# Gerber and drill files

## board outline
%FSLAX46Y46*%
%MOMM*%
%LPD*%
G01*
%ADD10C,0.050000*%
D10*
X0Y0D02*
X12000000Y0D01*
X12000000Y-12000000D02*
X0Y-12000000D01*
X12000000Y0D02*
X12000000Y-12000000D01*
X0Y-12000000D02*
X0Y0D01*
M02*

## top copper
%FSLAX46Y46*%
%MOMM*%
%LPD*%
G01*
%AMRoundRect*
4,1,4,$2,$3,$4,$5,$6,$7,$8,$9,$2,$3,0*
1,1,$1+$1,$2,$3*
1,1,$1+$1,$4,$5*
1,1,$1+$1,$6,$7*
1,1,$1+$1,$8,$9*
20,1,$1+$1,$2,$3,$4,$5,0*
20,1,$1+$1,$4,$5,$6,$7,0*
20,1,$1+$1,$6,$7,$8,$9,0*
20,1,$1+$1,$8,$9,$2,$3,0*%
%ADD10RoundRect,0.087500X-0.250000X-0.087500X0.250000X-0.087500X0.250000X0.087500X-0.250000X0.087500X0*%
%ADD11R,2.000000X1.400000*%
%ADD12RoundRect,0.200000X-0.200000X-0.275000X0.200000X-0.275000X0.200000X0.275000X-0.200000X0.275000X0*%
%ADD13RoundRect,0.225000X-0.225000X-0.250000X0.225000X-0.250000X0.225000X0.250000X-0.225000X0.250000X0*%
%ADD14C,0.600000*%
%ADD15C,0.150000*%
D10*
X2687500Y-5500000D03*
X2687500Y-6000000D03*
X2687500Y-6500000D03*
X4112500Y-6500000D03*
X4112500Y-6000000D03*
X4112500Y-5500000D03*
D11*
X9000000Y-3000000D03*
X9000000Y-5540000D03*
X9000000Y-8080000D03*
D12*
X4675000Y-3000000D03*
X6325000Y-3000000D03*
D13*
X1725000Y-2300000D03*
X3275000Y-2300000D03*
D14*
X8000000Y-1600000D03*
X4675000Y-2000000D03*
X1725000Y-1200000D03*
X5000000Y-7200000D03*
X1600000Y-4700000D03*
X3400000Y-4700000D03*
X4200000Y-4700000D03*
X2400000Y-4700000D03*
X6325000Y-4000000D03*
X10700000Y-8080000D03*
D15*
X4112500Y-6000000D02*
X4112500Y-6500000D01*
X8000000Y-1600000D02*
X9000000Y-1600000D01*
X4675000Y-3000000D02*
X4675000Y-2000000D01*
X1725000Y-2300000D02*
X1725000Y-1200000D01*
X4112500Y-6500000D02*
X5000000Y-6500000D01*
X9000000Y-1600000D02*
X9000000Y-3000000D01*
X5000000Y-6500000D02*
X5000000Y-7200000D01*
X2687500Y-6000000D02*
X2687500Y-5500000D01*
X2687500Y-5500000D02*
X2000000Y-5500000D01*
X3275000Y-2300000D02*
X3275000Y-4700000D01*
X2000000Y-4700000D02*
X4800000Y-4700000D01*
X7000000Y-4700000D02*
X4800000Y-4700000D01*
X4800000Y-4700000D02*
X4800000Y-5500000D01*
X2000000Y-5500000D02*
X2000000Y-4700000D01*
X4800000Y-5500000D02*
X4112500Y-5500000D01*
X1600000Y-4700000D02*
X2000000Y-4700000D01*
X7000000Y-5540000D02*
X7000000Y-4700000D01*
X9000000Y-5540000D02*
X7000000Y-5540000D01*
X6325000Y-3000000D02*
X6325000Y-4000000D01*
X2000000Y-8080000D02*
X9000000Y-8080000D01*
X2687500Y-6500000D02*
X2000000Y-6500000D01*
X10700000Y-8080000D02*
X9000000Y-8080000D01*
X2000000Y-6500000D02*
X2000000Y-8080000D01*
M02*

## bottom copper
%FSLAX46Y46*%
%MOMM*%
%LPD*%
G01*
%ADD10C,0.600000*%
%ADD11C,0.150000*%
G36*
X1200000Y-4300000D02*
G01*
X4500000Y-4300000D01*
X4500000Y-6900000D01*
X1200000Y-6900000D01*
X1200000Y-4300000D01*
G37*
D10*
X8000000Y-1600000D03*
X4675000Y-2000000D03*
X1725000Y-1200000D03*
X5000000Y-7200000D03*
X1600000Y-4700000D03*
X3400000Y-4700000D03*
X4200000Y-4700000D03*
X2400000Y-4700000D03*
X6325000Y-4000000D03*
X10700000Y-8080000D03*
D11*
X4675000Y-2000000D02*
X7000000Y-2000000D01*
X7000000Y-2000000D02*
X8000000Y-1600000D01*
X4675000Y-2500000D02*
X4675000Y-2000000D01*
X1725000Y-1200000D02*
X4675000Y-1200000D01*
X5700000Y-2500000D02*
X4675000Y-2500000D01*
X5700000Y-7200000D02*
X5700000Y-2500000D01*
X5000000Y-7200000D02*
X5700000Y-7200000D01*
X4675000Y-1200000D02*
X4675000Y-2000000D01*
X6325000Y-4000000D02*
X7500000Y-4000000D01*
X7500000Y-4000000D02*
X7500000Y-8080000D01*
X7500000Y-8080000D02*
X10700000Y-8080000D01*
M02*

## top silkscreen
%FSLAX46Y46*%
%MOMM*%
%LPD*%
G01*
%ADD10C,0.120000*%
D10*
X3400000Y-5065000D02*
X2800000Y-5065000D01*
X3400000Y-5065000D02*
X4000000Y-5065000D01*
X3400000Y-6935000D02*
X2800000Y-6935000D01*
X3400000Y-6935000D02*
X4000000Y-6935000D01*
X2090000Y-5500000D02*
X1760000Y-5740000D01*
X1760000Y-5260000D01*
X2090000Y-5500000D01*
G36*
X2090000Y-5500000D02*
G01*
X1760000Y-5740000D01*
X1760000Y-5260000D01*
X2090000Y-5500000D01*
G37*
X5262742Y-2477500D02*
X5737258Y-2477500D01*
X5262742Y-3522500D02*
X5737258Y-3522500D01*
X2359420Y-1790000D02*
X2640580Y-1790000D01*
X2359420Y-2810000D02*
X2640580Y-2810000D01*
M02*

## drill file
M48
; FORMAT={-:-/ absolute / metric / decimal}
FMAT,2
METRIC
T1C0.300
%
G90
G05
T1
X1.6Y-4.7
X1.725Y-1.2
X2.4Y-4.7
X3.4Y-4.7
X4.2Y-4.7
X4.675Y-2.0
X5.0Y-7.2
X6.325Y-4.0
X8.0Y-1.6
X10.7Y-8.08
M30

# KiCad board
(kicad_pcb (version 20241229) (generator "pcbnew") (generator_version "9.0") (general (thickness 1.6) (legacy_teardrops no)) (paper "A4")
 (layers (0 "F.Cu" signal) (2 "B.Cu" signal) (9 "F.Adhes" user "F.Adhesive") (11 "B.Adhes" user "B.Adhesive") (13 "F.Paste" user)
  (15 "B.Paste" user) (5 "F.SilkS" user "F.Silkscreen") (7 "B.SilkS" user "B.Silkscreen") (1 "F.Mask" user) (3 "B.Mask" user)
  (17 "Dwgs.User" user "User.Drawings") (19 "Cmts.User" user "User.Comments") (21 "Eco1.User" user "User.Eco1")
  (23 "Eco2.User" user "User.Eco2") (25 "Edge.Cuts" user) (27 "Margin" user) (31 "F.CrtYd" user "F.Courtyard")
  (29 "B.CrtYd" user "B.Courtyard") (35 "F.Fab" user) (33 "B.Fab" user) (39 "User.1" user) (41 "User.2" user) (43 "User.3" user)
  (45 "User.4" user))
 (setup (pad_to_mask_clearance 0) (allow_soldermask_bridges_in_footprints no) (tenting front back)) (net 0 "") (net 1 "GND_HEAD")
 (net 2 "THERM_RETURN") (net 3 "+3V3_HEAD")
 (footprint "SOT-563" (layer "F.Cu") (at 3.4 6)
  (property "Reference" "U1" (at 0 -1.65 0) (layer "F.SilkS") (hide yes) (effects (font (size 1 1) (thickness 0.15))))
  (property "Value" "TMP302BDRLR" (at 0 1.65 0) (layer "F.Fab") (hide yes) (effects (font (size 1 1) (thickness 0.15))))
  (fp_line (start 0 -0.935) (end -0.6 -0.935) (stroke (width 0.12) (type solid)) (layer "F.SilkS"))
  (fp_line (start 0 -0.935) (end 0.6 -0.935) (stroke (width 0.12) (type solid)) (layer "F.SilkS"))
  (fp_line (start 0 0.935) (end -0.6 0.935) (stroke (width 0.12) (type solid)) (layer "F.SilkS"))
  (fp_line (start 0 0.935) (end 0.6 0.935) (stroke (width 0.12) (type solid)) (layer "F.SilkS"))
  (fp_poly (pts (xy -1.31 -0.5) (xy -1.64 -0.26) (xy -1.64 -0.74)) (stroke (width 0.12) (type solid)) (fill yes) (layer "F.SilkS"))
  (pad "1" smd roundrect (at -0.7125 -0.5) (size 0.675 0.35) (layers "F.Cu" "F.Mask" "F.Paste") (roundrect_rratio 0.25) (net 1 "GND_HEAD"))
  (pad "2" smd roundrect (at -0.7125 0) (size 0.675 0.35) (layers "F.Cu" "F.Mask" "F.Paste") (roundrect_rratio 0.25) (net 1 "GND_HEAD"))
  (pad "3" smd roundrect (at -0.7125 0.5) (size 0.675 0.35) (layers "F.Cu" "F.Mask" "F.Paste") (roundrect_rratio 0.25)
   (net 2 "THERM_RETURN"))
  (pad "4" smd roundrect (at 0.7125 0.5) (size 0.675 0.35) (layers "F.Cu" "F.Mask" "F.Paste") (roundrect_rratio 0.25) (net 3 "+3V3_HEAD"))
  (pad "5" smd roundrect (at 0.7125 0) (size 0.675 0.35) (layers "F.Cu" "F.Mask" "F.Paste") (roundrect_rratio 0.25) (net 3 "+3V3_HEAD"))
  (pad "6" smd roundrect (at 0.7125 -0.5) (size 0.675 0.35) (layers "F.Cu" "F.Mask" "F.Paste") (roundrect_rratio 0.25) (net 1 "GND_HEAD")))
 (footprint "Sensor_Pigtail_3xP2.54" (layer "F.Cu") (at 9 3)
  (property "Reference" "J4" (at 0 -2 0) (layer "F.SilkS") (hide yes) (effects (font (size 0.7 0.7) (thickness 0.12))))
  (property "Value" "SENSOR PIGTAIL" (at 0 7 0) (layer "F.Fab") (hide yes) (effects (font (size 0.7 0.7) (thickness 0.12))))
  (pad "1" smd rect (at 0 0) (size 2 1.4) (layers "F.Cu" "F.Mask" "F.Paste") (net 3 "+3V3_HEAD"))
  (pad "2" smd rect (at 0 2.54) (size 2 1.4) (layers "F.Cu" "F.Mask" "F.Paste") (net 1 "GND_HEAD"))
  (pad "3" smd rect (at 0 5.08) (size 2 1.4) (layers "F.Cu" "F.Mask" "F.Paste") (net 2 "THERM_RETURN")))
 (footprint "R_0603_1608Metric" (layer "F.Cu") (at 5.5 3)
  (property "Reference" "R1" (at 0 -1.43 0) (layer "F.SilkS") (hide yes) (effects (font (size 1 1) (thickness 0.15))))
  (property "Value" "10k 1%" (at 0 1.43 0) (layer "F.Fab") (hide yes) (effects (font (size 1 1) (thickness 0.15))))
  (fp_line (start -0.237258 -0.5225) (end 0.237258 -0.5225) (stroke (width 0.12) (type solid)) (layer "F.SilkS"))
  (fp_line (start -0.237258 0.5225) (end 0.237258 0.5225) (stroke (width 0.12) (type solid)) (layer "F.SilkS"))
  (pad "1" smd roundrect (at -0.825 0) (size 0.8 0.95) (layers "F.Cu" "F.Mask" "F.Paste") (roundrect_rratio 0.25) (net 3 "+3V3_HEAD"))
  (pad "2" smd roundrect (at 0.825 0) (size 0.8 0.95) (layers "F.Cu" "F.Mask" "F.Paste") (roundrect_rratio 0.25) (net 2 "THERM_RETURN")))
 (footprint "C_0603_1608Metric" (layer "F.Cu") (at 2.5 2.3)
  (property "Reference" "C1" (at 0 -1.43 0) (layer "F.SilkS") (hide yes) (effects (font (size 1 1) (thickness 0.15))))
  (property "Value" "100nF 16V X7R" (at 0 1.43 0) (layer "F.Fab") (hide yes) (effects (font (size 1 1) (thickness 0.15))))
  (fp_line (start -0.14058 -0.51) (end 0.14058 -0.51) (stroke (width 0.12) (type solid)) (layer "F.SilkS"))
  (fp_line (start -0.14058 0.51) (end 0.14058 0.51) (stroke (width 0.12) (type solid)) (layer "F.SilkS"))
  (pad "1" smd roundrect (at -0.775 0) (size 0.9 0.95) (layers "F.Cu" "F.Mask" "F.Paste") (roundrect_rratio 0.25) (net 3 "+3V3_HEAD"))
  (pad "2" smd roundrect (at 0.775 0) (size 0.9 0.95) (layers "F.Cu" "F.Mask" "F.Paste") (roundrect_rratio 0.25) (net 1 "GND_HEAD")))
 (gr_rect (start 1.2 4.3) (end 4.5 6.9) (stroke (width 0) (type default)) (fill yes) (layer "B.Cu") (net 1))
 (gr_line (start 0 0) (end 12 0) (stroke (width 0.05) (type default)) (layer "Edge.Cuts"))
 (gr_line (start 12 12) (end 0 12) (stroke (width 0.05) (type default)) (layer "Edge.Cuts"))
 (gr_line (start 12 0) (end 12 12) (stroke (width 0.05) (type default)) (layer "Edge.Cuts"))
 (gr_line (start 0 12) (end 0 0) (stroke (width 0.05) (type default)) (layer "Edge.Cuts"))
 (segment (start 4.1125 6) (end 4.1125 6.5) (width 0.15) (layer "F.Cu") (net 3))
 (segment (start 8 1.6) (end 9 1.6) (width 0.15) (layer "F.Cu") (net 3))
 (segment (start 4.675 3) (end 4.675 2) (width 0.15) (layer "F.Cu") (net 3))
 (segment (start 1.725 2.3) (end 1.725 1.2) (width 0.15) (layer "F.Cu") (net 3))
 (segment (start 4.1125 6.5) (end 5 6.5) (width 0.15) (layer "F.Cu") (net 3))
 (segment (start 9 1.6) (end 9 3) (width 0.15) (layer "F.Cu") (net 3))
 (segment (start 5 6.5) (end 5 7.2) (width 0.15) (layer "F.Cu") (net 3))
 (via (at 8 1.6) (size 0.6) (drill 0.3) (layers "F.Cu" "B.Cu") (tenting front back) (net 3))
 (via (at 4.675 2) (size 0.6) (drill 0.3) (layers "F.Cu" "B.Cu") (tenting front back) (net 3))
 (via (at 1.725 1.2) (size 0.6) (drill 0.3) (layers "F.Cu" "B.Cu") (tenting front back) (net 3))
 (via (at 5 7.2) (size 0.6) (drill 0.3) (layers "F.Cu" "B.Cu") (tenting front back) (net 3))
 (segment (start 4.675 2) (end 7 2) (width 0.15) (layer "B.Cu") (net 3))
 (segment (start 7 2) (end 8 1.6) (width 0.15) (layer "B.Cu") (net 3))
 (segment (start 4.675 2.5) (end 4.675 2) (width 0.15) (layer "B.Cu") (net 3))
 (segment (start 1.725 1.2) (end 4.675 1.2) (width 0.15) (layer "B.Cu") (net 3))
 (segment (start 5.7 2.5) (end 4.675 2.5) (width 0.15) (layer "B.Cu") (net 3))
 (segment (start 5.7 7.2) (end 5.7 2.5) (width 0.15) (layer "B.Cu") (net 3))
 (segment (start 5 7.2) (end 5.7 7.2) (width 0.15) (layer "B.Cu") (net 3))
 (segment (start 4.675 1.2) (end 4.675 2) (width 0.15) (layer "B.Cu") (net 3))
 (segment (start 2.6875 6) (end 2.6875 5.5) (width 0.15) (layer "F.Cu") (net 1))
 (segment (start 2.6875 5.5) (end 2 5.5) (width 0.15) (layer "F.Cu") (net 1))
 (segment (start 3.275 2.3) (end 3.275 4.7) (width 0.15) (layer "F.Cu") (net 1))
 (segment (start 2 4.7) (end 4.8 4.7) (width 0.15) (layer "F.Cu") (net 1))
 (segment (start 7 4.7) (end 4.8 4.7) (width 0.15) (layer "F.Cu") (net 1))
 (segment (start 4.8 4.7) (end 4.8 5.5) (width 0.15) (layer "F.Cu") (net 1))
 (segment (start 2 5.5) (end 2 4.7) (width 0.15) (layer "F.Cu") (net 1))
 (segment (start 4.8 5.5) (end 4.1125 5.5) (width 0.15) (layer "F.Cu") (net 1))
 (segment (start 1.6 4.7) (end 2 4.7) (width 0.15) (layer "F.Cu") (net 1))
 (segment (start 7 5.54) (end 7 4.7) (width 0.15) (layer "F.Cu") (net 1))
 (segment (start 9 5.54) (end 7 5.54) (width 0.15) (layer "F.Cu") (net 1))
 (via (at 1.6 4.7) (size 0.6) (drill 0.3) (layers "F.Cu" "B.Cu") (tenting front back) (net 1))
 (via (at 3.4 4.7) (size 0.6) (drill 0.3) (layers "F.Cu" "B.Cu") (tenting front back) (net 1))
 (via (at 4.2 4.7) (size 0.6) (drill 0.3) (layers "F.Cu" "B.Cu") (tenting front back) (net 1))
 (via (at 2.4 4.7) (size 0.6) (drill 0.3) (layers "F.Cu" "B.Cu") (tenting front back) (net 1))
 (segment (start 6.325 3) (end 6.325 4) (width 0.15) (layer "F.Cu") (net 2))
 (segment (start 2 8.08) (end 9 8.08) (width 0.15) (layer "F.Cu") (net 2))
 (segment (start 2.6875 6.5) (end 2 6.5) (width 0.15) (layer "F.Cu") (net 2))
 (segment (start 10.7 8.08) (end 9 8.08) (width 0.15) (layer "F.Cu") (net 2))
 (segment (start 2 6.5) (end 2 8.08) (width 0.15) (layer "F.Cu") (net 2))
 (via (at 6.325 4) (size 0.6) (drill 0.3) (layers "F.Cu" "B.Cu") (tenting front back) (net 2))
 (via (at 10.7 8.08) (size 0.6) (drill 0.3) (layers "F.Cu" "B.Cu") (tenting front back) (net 2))
 (segment (start 6.325 4) (end 7.5 4) (width 0.15) (layer "B.Cu") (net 2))
 (segment (start 7.5 4) (end 7.5 8.08) (width 0.15) (layer "B.Cu") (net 2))
 (segment (start 7.5 8.08) (end 10.7 8.08) (width 0.15) (layer "B.Cu") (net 2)))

